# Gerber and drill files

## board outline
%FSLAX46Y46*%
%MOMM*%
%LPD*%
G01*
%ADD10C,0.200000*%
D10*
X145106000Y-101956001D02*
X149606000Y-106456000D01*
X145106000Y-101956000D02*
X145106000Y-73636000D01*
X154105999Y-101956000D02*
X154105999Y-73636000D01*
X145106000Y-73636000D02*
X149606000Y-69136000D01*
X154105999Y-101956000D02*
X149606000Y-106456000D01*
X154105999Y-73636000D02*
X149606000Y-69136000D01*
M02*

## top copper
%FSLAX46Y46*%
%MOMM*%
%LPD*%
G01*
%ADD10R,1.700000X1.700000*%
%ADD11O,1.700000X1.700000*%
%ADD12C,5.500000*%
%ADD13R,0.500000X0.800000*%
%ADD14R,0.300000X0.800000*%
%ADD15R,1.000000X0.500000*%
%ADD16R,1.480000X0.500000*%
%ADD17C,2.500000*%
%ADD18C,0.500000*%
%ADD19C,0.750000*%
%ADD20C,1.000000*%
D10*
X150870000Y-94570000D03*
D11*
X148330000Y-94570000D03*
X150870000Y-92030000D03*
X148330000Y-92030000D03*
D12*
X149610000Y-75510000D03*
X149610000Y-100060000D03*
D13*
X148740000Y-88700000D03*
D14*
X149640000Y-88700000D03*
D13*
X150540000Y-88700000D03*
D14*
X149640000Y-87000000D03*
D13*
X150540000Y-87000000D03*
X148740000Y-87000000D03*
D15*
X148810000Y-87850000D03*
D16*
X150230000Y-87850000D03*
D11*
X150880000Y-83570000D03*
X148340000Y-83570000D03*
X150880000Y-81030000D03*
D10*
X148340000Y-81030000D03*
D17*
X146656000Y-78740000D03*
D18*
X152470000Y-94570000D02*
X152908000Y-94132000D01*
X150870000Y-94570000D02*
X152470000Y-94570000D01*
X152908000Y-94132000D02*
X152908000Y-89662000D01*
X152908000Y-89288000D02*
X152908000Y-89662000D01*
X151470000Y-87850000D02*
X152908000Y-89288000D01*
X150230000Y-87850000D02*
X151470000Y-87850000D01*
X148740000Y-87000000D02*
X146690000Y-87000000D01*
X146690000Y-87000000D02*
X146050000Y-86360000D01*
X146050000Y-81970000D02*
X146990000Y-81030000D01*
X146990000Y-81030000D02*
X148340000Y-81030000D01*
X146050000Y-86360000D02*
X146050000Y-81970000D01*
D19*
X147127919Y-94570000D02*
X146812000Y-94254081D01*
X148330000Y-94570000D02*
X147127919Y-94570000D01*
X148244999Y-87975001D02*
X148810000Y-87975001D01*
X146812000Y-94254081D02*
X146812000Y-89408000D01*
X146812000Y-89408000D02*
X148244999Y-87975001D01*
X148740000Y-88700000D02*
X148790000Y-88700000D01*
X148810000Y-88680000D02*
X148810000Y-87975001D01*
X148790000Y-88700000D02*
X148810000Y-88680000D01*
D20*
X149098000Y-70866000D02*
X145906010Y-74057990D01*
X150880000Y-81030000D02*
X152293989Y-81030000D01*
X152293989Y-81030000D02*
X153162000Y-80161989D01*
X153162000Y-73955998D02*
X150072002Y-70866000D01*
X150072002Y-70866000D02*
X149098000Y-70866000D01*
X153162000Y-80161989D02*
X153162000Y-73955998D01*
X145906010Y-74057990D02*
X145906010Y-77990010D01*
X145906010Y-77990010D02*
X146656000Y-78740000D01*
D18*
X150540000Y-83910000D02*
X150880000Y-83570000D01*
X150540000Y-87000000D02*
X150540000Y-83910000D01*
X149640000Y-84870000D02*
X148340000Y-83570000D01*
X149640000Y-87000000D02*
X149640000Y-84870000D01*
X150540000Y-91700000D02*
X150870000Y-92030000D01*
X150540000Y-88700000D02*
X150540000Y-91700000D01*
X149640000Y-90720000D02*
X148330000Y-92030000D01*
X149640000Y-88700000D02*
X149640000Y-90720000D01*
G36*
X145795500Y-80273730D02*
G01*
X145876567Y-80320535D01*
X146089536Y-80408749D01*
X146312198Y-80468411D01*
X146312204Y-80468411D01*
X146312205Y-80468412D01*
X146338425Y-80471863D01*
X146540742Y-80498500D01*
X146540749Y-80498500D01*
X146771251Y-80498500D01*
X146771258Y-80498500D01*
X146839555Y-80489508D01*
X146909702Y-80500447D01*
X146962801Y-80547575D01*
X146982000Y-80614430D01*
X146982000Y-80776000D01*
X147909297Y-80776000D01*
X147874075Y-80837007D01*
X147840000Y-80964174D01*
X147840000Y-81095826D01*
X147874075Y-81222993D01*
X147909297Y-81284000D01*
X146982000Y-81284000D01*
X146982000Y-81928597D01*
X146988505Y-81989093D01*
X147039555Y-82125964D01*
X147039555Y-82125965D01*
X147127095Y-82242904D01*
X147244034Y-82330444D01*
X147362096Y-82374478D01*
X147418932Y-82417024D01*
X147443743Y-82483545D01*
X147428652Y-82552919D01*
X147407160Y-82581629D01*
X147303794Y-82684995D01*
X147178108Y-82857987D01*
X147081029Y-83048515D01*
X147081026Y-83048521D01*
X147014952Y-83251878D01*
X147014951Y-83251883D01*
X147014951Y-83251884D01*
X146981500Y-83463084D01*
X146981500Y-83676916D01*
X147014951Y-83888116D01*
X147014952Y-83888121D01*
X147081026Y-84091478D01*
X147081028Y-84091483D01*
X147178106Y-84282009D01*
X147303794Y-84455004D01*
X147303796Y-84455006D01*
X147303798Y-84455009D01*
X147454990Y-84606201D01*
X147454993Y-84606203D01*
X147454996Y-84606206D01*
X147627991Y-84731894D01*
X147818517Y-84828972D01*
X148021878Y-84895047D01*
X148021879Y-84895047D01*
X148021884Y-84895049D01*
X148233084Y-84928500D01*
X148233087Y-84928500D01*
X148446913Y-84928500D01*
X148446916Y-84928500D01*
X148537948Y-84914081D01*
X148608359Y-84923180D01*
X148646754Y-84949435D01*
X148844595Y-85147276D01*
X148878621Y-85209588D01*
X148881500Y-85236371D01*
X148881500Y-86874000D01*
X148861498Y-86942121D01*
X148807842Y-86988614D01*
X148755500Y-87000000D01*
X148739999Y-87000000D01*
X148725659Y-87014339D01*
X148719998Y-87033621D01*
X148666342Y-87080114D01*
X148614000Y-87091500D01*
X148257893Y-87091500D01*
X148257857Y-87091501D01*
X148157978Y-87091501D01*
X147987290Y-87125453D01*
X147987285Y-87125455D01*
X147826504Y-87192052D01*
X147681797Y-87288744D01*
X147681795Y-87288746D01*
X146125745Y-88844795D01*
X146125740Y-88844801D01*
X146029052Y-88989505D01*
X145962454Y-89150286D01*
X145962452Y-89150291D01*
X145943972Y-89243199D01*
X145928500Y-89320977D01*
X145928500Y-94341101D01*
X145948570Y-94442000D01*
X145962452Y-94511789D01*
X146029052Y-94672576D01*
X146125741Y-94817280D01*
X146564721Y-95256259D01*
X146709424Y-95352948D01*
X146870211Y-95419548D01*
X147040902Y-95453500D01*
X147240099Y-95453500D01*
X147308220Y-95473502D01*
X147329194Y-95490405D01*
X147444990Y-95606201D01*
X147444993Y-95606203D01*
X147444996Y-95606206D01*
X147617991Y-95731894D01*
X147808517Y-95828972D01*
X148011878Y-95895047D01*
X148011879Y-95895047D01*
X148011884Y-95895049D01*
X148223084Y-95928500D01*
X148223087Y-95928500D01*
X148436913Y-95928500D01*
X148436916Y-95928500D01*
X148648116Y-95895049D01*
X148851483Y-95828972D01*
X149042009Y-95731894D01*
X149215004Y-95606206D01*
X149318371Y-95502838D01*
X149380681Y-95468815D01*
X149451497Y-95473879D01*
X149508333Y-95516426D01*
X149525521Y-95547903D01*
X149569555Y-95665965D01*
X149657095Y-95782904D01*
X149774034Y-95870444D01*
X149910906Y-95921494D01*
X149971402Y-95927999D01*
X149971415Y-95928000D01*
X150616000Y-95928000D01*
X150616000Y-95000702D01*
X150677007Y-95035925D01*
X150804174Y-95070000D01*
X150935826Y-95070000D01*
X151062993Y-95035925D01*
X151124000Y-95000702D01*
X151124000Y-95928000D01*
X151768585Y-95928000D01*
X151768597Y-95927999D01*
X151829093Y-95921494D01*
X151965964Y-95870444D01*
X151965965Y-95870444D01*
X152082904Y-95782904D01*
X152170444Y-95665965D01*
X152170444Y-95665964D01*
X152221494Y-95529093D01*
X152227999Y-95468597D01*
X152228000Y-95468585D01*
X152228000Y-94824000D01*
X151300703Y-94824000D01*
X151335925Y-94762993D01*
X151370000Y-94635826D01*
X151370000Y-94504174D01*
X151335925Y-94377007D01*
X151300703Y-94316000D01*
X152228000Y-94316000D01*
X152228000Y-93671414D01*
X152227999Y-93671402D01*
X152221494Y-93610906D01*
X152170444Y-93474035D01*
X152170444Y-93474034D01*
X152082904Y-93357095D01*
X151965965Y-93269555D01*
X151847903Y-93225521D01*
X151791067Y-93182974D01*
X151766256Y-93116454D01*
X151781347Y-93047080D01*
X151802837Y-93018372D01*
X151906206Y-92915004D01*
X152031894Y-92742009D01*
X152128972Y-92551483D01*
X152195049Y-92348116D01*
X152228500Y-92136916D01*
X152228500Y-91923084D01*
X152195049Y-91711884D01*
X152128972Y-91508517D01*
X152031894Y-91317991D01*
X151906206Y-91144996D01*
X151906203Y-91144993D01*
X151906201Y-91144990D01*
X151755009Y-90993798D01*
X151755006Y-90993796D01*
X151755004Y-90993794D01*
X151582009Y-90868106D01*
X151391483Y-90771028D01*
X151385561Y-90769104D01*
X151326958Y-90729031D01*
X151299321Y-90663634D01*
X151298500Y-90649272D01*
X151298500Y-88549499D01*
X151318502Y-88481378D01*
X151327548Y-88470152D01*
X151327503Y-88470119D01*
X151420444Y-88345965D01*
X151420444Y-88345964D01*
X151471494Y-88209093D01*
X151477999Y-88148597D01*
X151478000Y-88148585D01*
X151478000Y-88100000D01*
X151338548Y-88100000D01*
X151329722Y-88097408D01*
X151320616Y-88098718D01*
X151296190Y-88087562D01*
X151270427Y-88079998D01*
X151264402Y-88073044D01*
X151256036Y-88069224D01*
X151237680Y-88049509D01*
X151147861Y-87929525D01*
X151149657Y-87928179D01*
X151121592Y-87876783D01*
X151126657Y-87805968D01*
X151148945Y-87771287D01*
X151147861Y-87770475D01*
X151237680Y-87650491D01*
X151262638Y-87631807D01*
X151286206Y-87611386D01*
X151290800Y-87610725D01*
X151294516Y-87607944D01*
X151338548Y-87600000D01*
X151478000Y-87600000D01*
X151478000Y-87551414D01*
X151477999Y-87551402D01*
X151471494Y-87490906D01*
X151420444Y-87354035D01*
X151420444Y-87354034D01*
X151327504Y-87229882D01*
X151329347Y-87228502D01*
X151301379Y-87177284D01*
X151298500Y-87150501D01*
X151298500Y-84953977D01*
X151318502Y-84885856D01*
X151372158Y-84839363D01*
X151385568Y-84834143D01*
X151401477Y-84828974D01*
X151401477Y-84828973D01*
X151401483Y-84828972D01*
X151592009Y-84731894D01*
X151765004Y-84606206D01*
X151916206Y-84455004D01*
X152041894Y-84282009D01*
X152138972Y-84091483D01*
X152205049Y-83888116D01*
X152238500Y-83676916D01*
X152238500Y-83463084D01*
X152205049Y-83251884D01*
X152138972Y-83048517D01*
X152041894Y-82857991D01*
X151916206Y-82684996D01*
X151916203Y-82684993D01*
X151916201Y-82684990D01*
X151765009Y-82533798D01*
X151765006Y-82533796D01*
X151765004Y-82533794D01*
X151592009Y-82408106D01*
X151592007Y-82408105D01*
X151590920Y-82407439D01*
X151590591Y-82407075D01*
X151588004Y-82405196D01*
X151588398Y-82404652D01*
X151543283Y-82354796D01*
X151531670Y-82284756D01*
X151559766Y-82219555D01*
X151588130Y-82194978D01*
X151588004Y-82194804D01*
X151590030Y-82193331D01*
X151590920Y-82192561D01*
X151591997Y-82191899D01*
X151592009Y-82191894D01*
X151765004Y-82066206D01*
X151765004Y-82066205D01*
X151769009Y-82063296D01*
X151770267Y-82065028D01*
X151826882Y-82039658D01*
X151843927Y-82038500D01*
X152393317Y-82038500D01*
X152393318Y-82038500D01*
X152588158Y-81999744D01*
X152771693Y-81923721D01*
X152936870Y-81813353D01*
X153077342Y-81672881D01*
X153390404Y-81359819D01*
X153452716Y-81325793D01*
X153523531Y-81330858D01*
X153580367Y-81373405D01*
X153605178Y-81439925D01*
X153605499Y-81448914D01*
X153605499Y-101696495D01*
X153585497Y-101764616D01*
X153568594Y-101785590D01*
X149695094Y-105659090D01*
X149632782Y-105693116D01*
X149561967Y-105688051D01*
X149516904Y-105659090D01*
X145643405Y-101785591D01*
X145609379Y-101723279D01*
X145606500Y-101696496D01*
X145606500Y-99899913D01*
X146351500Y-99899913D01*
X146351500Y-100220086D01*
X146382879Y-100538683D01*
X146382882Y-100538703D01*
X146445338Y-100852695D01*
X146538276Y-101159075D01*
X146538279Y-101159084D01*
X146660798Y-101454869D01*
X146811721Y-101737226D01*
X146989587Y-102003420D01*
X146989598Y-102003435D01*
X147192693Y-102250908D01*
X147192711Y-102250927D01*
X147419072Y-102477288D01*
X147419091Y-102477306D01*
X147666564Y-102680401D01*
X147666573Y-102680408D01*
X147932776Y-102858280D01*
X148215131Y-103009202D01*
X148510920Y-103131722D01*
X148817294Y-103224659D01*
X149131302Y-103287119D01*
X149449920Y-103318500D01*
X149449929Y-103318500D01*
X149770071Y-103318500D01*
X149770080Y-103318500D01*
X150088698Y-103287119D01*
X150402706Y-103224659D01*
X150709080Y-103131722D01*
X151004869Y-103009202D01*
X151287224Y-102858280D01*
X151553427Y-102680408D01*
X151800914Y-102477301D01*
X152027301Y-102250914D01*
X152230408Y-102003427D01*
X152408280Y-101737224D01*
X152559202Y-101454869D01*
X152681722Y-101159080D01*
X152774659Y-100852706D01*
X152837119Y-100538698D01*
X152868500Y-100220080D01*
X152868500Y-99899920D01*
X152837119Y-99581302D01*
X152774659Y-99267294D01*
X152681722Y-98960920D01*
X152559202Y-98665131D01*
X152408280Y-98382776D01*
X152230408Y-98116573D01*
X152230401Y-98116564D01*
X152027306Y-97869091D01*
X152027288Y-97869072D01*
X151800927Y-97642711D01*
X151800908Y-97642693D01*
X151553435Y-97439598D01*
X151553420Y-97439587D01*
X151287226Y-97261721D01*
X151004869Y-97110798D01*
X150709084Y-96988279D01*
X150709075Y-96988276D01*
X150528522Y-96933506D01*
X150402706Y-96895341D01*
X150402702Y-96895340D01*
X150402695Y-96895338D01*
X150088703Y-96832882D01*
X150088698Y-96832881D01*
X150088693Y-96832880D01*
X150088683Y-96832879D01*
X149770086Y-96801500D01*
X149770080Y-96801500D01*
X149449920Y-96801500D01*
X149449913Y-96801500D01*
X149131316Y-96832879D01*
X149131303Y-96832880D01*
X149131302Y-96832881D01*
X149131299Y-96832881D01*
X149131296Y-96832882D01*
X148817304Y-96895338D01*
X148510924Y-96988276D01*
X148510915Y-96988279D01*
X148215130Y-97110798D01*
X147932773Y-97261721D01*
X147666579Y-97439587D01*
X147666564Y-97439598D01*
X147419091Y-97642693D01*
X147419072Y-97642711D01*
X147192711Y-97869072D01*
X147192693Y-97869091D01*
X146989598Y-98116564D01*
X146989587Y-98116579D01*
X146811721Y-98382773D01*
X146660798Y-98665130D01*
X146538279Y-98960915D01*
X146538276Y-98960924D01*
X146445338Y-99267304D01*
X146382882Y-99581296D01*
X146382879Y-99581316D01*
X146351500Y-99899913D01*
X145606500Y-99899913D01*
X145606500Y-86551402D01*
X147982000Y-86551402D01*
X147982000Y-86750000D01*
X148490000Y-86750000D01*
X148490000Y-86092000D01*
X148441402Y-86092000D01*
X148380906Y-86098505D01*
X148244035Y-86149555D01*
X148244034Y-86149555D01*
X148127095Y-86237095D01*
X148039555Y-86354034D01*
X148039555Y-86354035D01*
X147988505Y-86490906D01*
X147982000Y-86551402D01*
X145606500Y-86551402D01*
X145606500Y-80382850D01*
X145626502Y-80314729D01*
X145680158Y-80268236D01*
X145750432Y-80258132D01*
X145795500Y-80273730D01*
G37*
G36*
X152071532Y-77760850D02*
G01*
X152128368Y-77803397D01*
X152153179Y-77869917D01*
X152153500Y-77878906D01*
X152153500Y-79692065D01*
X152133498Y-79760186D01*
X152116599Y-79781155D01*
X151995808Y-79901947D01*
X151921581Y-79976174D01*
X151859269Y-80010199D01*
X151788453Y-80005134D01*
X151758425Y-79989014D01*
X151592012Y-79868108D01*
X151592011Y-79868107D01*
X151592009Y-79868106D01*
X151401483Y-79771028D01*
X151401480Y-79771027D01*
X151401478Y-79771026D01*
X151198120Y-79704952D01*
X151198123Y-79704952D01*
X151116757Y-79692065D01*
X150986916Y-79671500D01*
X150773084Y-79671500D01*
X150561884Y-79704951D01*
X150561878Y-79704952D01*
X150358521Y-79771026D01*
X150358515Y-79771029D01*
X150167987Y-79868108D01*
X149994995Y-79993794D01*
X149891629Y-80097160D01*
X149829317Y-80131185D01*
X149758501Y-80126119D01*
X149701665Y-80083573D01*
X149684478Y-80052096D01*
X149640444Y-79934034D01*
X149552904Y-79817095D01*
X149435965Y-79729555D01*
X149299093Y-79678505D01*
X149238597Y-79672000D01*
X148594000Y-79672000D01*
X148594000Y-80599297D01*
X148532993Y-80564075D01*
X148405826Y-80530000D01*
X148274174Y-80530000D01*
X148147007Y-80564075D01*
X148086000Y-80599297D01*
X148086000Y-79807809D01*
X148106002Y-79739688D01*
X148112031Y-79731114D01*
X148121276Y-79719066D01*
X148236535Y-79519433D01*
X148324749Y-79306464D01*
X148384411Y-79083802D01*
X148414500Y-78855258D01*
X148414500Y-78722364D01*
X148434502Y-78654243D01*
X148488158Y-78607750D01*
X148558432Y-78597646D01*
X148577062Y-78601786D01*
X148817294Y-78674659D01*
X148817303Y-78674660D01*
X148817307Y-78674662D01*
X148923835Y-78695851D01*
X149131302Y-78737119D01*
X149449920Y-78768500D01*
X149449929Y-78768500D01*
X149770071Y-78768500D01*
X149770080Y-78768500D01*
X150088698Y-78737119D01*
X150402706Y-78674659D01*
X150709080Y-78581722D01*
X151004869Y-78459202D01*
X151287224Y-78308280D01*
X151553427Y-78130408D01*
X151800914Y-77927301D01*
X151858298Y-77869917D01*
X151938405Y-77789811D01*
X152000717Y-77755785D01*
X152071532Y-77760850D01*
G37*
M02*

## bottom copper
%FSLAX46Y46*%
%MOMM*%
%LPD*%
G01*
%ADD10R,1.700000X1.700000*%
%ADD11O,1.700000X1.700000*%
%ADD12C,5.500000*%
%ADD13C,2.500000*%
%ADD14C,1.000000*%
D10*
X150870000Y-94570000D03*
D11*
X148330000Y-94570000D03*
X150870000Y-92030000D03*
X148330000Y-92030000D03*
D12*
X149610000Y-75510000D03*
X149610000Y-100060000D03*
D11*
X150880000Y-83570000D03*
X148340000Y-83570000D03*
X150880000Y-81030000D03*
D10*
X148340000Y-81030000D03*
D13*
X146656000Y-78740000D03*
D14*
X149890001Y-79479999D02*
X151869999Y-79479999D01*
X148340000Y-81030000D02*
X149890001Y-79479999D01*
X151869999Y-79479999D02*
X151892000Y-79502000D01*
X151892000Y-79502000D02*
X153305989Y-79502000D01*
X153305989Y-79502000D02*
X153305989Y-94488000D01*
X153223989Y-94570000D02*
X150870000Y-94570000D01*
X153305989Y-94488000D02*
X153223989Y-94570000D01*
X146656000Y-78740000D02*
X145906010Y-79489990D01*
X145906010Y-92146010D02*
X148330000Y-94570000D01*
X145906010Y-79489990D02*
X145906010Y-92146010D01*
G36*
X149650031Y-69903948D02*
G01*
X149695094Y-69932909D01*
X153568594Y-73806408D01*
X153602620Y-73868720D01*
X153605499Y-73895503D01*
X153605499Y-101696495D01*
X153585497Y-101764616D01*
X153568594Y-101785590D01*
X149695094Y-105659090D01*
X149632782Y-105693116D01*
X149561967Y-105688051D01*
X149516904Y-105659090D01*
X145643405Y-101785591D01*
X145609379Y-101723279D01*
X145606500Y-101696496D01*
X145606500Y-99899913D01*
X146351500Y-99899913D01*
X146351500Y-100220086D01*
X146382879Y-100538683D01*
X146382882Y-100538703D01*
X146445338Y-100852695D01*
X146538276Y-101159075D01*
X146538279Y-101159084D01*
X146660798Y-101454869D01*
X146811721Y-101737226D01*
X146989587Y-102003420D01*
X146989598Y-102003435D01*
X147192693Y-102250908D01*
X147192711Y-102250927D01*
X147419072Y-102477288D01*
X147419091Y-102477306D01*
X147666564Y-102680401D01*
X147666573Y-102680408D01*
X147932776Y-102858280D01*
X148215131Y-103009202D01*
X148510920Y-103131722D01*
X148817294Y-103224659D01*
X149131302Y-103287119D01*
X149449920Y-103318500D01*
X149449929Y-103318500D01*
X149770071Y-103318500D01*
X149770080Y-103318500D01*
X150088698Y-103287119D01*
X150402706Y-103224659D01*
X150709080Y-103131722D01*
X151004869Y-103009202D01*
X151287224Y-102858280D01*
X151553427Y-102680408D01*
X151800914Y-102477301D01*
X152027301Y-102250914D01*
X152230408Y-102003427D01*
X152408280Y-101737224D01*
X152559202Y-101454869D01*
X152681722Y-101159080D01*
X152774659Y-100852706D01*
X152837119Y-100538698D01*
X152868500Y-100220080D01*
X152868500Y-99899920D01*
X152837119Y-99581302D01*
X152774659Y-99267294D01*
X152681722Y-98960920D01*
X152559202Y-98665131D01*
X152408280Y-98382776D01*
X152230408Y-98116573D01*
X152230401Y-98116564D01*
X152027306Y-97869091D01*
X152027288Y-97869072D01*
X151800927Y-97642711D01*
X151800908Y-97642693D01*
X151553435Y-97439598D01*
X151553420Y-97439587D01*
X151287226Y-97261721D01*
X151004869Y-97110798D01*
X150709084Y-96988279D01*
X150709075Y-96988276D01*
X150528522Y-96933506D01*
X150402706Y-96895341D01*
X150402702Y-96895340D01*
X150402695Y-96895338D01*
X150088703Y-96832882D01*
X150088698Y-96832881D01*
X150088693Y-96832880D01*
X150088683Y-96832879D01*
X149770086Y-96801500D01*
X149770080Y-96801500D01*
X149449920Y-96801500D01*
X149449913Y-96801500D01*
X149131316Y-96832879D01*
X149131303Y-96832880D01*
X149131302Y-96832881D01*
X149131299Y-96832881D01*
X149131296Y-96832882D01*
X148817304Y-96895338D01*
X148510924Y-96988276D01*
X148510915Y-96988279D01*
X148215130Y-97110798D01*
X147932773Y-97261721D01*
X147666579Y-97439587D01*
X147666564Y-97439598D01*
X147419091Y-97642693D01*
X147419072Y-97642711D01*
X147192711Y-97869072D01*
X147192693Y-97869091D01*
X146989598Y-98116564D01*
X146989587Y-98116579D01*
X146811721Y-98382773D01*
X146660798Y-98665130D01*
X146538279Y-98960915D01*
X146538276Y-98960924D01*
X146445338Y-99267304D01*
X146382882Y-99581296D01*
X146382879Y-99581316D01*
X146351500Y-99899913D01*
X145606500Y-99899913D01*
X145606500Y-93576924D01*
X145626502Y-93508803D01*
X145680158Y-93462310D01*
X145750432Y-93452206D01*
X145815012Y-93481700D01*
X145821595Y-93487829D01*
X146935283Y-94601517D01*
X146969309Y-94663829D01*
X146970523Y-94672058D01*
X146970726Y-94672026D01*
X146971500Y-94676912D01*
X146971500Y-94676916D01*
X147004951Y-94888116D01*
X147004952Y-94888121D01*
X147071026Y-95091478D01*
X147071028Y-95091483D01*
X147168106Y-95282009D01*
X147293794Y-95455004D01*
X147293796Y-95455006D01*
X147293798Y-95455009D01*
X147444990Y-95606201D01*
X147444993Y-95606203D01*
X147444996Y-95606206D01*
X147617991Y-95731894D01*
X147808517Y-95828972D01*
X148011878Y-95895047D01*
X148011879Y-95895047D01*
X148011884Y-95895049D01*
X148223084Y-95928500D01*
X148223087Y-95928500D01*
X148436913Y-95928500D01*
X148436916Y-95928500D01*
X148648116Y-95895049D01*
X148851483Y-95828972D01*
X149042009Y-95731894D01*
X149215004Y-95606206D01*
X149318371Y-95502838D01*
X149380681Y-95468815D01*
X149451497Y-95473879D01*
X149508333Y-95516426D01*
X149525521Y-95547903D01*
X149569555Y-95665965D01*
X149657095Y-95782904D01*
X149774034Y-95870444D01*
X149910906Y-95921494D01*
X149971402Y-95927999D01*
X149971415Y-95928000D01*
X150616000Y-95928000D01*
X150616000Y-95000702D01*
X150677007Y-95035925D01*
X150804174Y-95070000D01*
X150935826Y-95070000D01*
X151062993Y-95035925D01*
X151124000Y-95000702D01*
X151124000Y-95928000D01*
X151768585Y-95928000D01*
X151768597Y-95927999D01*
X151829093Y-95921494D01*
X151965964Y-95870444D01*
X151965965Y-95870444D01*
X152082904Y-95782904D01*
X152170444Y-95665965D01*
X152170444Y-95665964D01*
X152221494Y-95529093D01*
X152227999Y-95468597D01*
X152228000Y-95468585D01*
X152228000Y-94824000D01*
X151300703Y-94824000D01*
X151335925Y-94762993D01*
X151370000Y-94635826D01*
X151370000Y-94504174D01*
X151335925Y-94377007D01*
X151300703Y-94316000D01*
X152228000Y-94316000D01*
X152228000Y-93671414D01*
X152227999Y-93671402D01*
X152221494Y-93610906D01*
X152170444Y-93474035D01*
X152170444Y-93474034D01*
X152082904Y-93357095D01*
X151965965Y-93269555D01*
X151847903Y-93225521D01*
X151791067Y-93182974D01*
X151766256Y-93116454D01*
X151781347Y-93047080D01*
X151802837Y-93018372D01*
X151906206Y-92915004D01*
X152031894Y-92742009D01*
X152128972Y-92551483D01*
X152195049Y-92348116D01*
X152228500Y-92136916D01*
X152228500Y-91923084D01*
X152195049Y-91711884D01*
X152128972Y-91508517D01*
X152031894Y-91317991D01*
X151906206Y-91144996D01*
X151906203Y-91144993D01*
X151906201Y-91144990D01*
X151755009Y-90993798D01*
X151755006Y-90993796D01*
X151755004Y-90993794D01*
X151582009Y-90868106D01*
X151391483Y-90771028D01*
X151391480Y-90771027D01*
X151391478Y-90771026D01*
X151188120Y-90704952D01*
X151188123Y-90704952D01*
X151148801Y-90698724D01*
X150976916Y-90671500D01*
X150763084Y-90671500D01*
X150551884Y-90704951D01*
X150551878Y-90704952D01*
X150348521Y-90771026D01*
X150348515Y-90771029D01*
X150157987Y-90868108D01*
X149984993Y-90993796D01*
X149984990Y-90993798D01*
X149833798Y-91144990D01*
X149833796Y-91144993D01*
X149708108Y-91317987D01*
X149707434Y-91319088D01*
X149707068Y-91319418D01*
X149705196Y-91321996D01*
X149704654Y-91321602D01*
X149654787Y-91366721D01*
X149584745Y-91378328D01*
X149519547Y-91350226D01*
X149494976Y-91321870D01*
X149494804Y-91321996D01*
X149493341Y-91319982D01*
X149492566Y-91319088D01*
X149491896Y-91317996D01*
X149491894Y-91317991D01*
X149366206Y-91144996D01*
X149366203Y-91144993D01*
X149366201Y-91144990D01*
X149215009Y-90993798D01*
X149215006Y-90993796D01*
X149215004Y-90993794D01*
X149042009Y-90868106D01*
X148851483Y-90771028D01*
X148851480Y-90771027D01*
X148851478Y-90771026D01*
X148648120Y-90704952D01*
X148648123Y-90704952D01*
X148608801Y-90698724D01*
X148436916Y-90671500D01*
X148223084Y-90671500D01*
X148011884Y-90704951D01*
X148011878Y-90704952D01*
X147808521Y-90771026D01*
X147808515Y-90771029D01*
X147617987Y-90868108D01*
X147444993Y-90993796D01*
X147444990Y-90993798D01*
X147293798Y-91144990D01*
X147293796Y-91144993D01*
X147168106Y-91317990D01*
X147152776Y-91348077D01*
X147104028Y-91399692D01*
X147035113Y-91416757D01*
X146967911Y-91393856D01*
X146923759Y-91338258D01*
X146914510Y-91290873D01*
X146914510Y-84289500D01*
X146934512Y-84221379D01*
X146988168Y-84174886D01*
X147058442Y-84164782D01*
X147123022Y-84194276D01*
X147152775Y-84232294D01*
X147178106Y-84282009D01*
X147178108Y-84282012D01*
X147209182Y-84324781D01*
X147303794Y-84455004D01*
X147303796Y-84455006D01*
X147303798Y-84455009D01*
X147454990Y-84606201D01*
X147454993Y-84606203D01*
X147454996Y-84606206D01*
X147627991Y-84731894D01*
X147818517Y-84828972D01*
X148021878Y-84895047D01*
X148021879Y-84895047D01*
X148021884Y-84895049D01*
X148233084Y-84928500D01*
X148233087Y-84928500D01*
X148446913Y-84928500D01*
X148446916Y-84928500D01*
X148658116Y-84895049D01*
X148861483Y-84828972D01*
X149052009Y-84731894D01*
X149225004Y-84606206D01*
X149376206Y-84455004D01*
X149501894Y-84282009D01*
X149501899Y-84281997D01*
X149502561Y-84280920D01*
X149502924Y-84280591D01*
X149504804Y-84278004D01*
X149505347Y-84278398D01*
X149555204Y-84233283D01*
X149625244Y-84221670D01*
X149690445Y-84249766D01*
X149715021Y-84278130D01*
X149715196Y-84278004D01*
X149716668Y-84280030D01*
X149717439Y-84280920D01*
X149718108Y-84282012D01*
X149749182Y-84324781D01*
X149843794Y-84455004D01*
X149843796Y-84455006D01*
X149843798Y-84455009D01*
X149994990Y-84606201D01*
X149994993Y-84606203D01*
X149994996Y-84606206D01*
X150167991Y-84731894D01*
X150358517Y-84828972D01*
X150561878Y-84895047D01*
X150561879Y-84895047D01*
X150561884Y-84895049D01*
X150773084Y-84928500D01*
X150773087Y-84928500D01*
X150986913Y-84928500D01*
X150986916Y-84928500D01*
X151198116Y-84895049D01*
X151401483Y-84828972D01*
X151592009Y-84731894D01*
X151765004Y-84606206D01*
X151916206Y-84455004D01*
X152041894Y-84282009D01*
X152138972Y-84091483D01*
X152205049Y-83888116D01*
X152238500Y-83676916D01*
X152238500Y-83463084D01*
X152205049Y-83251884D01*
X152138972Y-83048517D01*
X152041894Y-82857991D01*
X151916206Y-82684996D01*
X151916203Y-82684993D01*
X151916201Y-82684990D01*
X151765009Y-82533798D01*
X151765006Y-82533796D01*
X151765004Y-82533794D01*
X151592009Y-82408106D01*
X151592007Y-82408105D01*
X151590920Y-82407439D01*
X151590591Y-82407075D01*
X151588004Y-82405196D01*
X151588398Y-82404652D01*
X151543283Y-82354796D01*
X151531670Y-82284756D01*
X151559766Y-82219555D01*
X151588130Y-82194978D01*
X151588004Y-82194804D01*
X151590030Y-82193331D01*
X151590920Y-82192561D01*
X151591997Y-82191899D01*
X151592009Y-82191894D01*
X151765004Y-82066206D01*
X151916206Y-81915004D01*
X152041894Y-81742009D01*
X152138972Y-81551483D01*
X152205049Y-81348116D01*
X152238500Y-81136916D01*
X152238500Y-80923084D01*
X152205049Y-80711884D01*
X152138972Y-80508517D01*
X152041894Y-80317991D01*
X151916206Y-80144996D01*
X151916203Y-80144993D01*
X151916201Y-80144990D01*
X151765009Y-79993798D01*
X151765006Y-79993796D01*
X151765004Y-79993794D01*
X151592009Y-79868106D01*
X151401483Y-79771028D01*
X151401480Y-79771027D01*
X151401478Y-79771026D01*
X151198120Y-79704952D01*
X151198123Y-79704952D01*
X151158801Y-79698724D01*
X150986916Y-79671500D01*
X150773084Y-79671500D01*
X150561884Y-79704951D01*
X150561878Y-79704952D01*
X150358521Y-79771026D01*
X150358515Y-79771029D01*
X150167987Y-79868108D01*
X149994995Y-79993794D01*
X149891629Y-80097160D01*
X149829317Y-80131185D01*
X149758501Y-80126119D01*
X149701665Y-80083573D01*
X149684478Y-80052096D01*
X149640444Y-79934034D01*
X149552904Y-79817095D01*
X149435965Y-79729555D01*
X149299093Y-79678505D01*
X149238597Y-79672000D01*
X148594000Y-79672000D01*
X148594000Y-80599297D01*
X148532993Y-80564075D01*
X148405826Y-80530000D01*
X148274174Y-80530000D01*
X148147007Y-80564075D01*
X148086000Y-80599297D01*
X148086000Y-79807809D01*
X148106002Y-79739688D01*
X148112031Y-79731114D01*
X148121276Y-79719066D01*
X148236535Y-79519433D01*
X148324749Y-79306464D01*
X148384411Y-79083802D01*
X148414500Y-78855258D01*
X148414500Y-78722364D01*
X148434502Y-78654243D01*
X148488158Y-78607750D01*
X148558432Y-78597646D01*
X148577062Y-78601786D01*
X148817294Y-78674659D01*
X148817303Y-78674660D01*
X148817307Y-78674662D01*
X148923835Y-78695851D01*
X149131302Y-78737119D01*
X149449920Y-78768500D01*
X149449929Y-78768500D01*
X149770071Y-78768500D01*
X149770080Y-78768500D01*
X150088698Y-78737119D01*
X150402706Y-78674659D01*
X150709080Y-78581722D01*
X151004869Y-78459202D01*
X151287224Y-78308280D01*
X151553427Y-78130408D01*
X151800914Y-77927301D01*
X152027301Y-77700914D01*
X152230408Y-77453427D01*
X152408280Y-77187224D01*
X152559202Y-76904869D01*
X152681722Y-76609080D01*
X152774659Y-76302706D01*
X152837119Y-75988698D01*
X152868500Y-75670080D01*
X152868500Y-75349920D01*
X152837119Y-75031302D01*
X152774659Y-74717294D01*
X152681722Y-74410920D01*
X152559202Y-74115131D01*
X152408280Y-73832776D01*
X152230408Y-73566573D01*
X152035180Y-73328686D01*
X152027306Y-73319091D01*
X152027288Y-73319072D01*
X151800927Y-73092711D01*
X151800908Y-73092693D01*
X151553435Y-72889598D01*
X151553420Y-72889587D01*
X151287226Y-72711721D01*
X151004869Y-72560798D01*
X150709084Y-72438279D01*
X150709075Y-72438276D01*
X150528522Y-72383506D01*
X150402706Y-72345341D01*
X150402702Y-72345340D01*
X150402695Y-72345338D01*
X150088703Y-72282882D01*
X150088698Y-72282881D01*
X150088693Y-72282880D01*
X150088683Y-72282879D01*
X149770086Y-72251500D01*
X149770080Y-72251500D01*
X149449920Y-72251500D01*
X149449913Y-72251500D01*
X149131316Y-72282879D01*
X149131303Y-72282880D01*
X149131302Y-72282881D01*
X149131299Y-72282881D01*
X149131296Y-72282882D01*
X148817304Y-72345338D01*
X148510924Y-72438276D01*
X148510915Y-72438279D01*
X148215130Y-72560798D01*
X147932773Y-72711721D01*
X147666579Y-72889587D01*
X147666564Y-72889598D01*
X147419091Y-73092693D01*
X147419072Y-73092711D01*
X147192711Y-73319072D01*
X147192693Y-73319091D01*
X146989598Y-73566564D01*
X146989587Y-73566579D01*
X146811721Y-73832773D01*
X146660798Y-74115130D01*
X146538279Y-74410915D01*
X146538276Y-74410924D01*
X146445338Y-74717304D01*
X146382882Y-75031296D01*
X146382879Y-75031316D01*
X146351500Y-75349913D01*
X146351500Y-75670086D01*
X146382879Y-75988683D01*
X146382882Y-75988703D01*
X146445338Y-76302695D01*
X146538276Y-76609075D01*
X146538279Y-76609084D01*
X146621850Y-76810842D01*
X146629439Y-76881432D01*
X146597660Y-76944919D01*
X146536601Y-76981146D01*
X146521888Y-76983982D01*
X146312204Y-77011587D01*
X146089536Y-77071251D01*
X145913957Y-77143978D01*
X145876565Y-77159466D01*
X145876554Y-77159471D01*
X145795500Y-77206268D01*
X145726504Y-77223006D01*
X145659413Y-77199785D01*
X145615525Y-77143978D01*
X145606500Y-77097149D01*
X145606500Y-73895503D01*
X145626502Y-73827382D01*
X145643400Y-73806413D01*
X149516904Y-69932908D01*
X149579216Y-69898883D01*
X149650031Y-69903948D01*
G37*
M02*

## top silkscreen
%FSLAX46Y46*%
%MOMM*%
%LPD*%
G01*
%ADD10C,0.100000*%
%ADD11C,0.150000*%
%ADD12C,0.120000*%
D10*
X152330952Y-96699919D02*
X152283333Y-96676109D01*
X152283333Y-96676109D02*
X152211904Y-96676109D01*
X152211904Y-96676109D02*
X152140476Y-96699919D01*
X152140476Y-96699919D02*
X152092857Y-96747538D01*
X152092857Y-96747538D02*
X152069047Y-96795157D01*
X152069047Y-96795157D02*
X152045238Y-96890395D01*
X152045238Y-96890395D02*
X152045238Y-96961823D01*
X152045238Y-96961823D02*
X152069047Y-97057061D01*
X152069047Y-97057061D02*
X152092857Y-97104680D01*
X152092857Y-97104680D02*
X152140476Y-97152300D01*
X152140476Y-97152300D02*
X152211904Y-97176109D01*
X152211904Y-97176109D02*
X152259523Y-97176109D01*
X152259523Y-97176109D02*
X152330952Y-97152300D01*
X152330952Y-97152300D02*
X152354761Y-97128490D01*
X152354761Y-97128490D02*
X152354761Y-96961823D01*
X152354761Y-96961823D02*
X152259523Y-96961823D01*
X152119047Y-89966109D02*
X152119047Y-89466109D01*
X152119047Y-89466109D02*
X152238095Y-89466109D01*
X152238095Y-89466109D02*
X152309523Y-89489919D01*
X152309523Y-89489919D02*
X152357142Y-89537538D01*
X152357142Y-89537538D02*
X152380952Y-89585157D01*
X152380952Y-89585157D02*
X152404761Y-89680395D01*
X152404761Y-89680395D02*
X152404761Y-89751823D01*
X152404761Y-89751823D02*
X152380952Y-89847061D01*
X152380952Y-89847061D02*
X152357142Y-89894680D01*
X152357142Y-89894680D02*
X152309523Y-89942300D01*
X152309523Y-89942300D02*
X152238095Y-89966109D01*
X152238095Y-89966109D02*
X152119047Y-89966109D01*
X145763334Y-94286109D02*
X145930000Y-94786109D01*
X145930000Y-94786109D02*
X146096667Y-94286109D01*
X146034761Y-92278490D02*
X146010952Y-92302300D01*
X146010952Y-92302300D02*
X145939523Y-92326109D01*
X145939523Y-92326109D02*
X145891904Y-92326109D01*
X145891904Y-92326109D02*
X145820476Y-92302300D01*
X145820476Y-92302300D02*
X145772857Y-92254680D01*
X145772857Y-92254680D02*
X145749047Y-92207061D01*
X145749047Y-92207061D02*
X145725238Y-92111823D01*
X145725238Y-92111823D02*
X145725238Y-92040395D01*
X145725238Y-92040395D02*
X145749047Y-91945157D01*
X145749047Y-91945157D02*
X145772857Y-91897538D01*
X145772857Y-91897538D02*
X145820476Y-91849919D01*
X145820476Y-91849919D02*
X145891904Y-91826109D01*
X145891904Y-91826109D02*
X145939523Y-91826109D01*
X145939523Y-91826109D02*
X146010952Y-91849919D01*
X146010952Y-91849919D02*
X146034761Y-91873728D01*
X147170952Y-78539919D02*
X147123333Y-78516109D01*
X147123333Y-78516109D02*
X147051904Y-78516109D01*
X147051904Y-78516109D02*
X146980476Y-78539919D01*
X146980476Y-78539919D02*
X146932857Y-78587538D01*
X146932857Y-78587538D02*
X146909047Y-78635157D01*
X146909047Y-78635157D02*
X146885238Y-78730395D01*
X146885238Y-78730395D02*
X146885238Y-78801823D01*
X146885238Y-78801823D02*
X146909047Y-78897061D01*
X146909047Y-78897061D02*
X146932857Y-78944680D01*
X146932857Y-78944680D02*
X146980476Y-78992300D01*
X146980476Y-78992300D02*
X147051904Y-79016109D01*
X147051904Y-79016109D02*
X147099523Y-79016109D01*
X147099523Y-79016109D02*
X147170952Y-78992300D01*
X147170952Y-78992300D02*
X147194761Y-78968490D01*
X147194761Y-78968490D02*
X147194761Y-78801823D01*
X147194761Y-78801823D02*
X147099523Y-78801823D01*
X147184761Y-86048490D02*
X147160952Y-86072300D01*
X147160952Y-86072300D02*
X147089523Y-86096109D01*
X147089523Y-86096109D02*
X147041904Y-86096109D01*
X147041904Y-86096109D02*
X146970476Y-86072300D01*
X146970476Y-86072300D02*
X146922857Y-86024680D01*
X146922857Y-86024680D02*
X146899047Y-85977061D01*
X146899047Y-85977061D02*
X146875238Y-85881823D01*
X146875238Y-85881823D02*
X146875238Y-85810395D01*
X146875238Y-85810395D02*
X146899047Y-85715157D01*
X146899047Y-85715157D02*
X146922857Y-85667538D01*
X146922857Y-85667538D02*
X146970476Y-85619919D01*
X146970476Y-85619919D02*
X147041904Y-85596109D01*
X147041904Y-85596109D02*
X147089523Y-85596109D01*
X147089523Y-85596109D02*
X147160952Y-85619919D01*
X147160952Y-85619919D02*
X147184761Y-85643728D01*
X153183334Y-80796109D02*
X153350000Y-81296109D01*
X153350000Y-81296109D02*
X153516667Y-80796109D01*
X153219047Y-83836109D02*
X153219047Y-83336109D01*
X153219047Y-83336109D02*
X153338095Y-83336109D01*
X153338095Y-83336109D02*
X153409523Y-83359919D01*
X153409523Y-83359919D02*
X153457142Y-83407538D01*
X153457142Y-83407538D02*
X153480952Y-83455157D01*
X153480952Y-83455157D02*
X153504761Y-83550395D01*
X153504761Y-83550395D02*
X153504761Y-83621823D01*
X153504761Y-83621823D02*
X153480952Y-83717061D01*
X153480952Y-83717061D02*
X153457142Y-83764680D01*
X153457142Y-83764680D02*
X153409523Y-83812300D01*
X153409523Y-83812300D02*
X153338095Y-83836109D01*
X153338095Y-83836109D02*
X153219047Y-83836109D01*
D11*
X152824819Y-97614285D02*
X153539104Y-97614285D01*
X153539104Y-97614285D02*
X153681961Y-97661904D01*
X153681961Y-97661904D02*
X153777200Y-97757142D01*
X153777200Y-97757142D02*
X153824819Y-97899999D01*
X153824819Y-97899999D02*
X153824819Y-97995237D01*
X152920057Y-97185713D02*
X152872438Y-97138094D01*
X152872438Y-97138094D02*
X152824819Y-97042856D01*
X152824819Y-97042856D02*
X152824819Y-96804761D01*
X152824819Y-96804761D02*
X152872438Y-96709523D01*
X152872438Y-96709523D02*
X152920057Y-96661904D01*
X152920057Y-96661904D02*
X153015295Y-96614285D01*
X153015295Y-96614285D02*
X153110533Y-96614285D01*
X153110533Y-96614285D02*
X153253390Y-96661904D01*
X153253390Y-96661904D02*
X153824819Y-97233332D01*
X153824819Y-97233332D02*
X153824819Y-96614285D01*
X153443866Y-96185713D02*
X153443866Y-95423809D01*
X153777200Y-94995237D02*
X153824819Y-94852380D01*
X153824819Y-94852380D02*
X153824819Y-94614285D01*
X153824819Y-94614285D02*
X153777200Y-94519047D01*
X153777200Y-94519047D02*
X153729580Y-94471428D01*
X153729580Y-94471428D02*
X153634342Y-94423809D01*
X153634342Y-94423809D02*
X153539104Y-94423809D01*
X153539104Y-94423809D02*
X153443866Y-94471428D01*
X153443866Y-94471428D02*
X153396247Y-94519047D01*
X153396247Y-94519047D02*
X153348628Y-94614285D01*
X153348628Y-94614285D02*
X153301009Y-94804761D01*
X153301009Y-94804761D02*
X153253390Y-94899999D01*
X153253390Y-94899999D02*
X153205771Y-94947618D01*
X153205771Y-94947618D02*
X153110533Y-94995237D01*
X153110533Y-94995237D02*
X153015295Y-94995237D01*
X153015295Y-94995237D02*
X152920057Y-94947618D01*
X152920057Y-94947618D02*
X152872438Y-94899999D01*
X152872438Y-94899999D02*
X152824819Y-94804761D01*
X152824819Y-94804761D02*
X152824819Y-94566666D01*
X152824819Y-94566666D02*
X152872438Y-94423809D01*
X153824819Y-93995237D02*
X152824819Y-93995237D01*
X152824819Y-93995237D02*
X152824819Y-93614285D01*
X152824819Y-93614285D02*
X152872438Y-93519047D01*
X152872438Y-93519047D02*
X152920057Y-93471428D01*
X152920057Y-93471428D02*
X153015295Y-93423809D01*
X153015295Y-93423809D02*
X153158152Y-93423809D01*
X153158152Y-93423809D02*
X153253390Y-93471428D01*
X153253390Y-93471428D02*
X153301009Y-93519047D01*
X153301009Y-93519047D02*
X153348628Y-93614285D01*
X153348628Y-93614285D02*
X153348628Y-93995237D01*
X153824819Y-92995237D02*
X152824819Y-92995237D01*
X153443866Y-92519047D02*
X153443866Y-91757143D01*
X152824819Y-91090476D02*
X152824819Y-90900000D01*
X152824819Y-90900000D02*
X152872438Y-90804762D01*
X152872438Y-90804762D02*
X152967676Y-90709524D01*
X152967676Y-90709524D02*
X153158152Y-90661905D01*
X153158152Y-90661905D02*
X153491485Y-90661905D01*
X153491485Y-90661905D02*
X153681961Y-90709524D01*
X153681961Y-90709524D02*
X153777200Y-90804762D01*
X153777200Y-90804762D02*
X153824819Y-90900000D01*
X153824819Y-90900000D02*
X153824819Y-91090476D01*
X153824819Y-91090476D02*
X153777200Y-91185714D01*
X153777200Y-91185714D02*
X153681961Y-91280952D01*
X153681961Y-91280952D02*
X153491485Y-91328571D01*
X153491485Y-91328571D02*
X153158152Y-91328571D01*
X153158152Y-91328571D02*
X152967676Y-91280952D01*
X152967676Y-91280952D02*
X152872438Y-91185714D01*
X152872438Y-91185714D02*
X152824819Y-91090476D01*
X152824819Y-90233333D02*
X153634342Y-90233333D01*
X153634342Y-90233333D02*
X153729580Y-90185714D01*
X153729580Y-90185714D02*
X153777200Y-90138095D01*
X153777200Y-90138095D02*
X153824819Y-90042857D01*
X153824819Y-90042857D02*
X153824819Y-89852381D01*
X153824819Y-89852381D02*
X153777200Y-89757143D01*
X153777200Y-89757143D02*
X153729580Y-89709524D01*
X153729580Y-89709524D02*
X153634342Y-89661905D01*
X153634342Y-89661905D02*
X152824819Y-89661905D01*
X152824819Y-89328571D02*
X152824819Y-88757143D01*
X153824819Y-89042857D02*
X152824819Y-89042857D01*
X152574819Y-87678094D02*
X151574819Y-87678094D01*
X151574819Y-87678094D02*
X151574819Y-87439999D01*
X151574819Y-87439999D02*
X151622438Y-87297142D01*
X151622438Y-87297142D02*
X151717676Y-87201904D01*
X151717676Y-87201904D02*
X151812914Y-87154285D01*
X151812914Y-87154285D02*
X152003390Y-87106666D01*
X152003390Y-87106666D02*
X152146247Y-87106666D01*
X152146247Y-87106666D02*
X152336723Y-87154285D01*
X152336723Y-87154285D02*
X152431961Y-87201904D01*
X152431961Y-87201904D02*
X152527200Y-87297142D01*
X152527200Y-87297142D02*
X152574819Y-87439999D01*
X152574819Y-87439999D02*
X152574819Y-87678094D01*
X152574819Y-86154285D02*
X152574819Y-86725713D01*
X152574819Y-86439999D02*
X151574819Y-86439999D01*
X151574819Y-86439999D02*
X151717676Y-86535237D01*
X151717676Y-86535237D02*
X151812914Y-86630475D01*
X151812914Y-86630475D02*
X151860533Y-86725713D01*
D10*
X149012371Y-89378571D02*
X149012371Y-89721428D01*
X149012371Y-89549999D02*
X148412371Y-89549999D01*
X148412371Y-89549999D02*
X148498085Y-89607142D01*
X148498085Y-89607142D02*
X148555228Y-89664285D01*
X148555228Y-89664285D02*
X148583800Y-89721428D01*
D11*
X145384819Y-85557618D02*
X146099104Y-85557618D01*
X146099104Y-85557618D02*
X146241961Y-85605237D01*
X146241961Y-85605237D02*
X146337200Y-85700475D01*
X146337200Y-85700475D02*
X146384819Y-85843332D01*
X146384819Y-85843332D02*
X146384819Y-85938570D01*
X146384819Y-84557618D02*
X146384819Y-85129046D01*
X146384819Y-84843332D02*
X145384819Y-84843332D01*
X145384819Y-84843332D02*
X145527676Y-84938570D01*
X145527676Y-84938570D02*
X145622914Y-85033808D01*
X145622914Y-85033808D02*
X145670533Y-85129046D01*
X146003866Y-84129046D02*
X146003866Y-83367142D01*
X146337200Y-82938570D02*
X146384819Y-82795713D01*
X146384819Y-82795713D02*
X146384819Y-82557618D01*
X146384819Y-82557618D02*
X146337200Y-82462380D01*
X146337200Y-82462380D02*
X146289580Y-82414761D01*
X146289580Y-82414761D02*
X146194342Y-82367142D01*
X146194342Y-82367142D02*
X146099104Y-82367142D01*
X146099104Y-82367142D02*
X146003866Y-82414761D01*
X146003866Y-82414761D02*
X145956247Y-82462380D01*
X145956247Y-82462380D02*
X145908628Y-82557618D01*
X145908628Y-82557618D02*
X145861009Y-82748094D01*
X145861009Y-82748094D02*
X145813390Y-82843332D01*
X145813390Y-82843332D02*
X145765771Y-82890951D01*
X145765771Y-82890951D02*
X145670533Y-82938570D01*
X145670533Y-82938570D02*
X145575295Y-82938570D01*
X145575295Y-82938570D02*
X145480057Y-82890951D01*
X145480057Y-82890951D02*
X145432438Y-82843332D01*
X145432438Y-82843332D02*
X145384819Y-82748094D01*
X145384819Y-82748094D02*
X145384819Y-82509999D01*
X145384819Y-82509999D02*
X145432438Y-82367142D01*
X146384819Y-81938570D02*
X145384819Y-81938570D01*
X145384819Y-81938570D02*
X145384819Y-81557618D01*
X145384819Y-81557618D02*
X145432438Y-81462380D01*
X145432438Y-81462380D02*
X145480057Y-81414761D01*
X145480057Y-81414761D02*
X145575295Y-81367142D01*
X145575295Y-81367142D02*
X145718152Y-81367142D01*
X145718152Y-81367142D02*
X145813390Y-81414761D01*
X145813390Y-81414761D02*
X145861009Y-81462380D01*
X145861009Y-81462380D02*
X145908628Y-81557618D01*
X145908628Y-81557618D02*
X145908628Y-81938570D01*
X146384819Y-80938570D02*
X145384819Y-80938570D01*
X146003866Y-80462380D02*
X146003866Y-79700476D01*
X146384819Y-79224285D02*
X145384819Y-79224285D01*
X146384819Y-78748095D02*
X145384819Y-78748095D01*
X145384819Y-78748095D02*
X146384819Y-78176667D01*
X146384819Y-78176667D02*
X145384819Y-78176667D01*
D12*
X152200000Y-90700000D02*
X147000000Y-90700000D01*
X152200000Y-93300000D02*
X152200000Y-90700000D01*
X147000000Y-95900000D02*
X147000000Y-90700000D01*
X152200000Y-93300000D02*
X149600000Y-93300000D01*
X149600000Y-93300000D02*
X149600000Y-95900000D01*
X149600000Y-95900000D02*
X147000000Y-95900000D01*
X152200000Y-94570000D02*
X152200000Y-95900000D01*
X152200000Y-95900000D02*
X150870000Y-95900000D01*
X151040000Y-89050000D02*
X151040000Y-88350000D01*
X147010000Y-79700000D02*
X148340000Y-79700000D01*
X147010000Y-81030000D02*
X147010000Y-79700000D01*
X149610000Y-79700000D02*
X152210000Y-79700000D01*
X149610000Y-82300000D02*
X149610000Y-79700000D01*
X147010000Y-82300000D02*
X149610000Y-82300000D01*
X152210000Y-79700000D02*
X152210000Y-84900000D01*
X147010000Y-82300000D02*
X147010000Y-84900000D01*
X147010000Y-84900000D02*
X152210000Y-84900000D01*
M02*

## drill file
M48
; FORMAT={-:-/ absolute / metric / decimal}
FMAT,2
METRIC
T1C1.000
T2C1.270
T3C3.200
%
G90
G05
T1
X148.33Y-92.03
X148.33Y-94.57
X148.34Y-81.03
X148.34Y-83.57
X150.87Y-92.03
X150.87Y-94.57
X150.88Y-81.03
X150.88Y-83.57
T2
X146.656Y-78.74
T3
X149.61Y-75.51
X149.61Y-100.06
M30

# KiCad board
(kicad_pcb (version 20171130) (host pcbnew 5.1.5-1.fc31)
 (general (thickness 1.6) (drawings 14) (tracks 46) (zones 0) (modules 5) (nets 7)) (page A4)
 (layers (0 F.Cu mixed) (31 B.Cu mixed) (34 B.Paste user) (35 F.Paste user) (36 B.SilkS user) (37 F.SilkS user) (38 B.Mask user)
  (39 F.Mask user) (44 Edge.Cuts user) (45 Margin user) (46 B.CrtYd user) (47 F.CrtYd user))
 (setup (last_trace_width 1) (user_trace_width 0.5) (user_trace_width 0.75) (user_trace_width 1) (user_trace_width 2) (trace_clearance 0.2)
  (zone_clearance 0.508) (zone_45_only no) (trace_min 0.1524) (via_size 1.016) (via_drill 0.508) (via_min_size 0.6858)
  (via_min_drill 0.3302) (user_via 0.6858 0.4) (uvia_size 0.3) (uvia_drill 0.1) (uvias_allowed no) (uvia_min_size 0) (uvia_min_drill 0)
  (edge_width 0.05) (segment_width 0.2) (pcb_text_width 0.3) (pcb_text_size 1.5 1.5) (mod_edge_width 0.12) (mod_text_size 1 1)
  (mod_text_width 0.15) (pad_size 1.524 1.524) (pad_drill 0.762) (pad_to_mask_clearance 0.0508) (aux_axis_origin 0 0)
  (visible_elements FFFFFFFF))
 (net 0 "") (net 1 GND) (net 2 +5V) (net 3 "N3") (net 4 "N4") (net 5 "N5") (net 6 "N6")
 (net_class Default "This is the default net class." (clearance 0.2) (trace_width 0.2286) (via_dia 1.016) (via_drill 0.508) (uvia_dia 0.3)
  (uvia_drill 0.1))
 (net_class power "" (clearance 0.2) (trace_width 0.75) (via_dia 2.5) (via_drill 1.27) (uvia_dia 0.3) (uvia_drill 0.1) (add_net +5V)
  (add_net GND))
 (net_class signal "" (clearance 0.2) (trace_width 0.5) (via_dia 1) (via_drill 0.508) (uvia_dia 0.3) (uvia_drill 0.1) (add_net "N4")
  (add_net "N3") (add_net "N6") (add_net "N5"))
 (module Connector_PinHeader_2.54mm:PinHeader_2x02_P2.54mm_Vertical (layer F.Cu) (at 150.87 94.57 180)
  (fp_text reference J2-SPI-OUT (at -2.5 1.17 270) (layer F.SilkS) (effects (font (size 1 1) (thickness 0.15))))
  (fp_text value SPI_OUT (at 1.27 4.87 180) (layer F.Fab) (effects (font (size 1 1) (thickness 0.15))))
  (fp_line (start -1.33 3.87) (end 3.87 3.87) (layer F.SilkS) (width 0.12))
  (fp_line (start -1.33 1.27) (end -1.33 3.87) (layer F.SilkS) (width 0.12))
  (fp_line (start 3.87 -1.33) (end 3.87 3.87) (layer F.SilkS) (width 0.12))
  (fp_line (start -1.33 1.27) (end 1.27 1.27) (layer F.SilkS) (width 0.12))
  (fp_line (start 1.27 1.27) (end 1.27 -1.33) (layer F.SilkS) (width 0.12))
  (fp_line (start 1.27 -1.33) (end 3.87 -1.33) (layer F.SilkS) (width 0.12))
  (fp_line (start -1.33 0) (end -1.33 -1.33) (layer F.SilkS) (width 0.12))
  (fp_line (start -1.33 -1.33) (end 0 -1.33) (layer F.SilkS) (width 0.12))
  (pad 1 thru_hole rect (at 0 0 180) (size 1.7 1.7) (drill 1) (layers *.Cu *.Mask) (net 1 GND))
  (pad 2 thru_hole oval (at 2.54 0 180) (size 1.7 1.7) (drill 1) (layers *.Cu *.Mask) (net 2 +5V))
  (pad 3 thru_hole oval (at 0 2.54 180) (size 1.7 1.7) (drill 1) (layers *.Cu *.Mask) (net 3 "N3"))
  (pad 4 thru_hole oval (at 2.54 2.54 180) (size 1.7 1.7) (drill 1) (layers *.Cu *.Mask) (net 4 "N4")))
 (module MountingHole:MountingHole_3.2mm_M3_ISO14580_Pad (layer F.Cu) (at 149.61 75.51)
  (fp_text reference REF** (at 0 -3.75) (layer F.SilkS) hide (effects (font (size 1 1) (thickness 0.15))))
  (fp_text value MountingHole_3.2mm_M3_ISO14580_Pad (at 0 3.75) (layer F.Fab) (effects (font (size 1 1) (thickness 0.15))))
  (pad 1 thru_hole circle (at 0 0) (size 5.5 5.5) (drill 3.2) (layers *.Cu *.Mask)))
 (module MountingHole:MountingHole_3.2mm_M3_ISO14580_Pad (layer F.Cu) (at 149.61 100.06)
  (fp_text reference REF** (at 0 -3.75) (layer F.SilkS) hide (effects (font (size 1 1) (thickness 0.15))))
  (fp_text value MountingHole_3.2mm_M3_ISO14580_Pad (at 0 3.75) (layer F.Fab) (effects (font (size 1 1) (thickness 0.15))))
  (pad 1 thru_hole circle (at 0 0) (size 5.5 5.5) (drill 3.2) (layers *.Cu *.Mask)))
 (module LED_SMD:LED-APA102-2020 (layer F.Cu) (at 149.64 87.85 90)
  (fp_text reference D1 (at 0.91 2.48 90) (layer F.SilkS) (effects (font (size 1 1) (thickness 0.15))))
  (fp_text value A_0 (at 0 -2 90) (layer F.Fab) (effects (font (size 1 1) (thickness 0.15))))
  (fp_line (start -1.2 1.4) (end -0.5 1.4) (layer F.SilkS) (width 0.12))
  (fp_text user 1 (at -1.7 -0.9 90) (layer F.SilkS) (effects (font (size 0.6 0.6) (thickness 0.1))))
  (pad 1 smd rect (at -0.85 -0.9 90) (size 0.8 0.5) (layers F.Cu F.Paste F.Mask) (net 2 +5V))
  (pad 2 smd rect (at -0.85 0 90) (size 0.8 0.3) (layers F.Cu F.Paste F.Mask) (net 4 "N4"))
  (pad 3 smd rect (at -0.85 0.9 90) (size 0.8 0.5) (layers F.Cu F.Paste F.Mask) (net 3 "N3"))
  (pad 5 smd rect (at 0.85 0 90) (size 0.8 0.3) (layers F.Cu F.Paste F.Mask) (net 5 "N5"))
  (pad 4 smd rect (at 0.85 0.9 90) (size 0.8 0.5) (layers F.Cu F.Paste F.Mask) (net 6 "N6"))
  (pad 6 smd rect (at 0.85 -0.9 90) (size 0.8 0.5) (layers F.Cu F.Paste F.Mask) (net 1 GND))
  (pad 1 smd rect (at 0 -0.83 180) (size 1 0.5) (layers F.Cu F.Paste F.Mask) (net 2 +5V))
  (pad 6 smd rect (at 0 0.59 180) (size 1.48 0.5) (layers F.Cu F.Paste F.Mask) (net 1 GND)))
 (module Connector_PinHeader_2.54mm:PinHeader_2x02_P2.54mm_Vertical (layer F.Cu) (at 148.34 81.03)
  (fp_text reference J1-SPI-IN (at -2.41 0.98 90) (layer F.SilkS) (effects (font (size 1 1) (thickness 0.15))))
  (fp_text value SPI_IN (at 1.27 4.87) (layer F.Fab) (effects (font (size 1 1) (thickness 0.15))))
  (fp_line (start -1.33 -1.33) (end 0 -1.33) (layer F.SilkS) (width 0.12))
  (fp_line (start -1.33 0) (end -1.33 -1.33) (layer F.SilkS) (width 0.12))
  (fp_line (start 1.27 -1.33) (end 3.87 -1.33) (layer F.SilkS) (width 0.12))
  (fp_line (start 1.27 1.27) (end 1.27 -1.33) (layer F.SilkS) (width 0.12))
  (fp_line (start -1.33 1.27) (end 1.27 1.27) (layer F.SilkS) (width 0.12))
  (fp_line (start 3.87 -1.33) (end 3.87 3.87) (layer F.SilkS) (width 0.12))
  (fp_line (start -1.33 1.27) (end -1.33 3.87) (layer F.SilkS) (width 0.12))
  (fp_line (start -1.33 3.87) (end 3.87 3.87) (layer F.SilkS) (width 0.12))
  (pad 4 thru_hole oval (at 2.54 2.54) (size 1.7 1.7) (drill 1) (layers *.Cu *.Mask) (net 6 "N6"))
  (pad 3 thru_hole oval (at 0 2.54) (size 1.7 1.7) (drill 1) (layers *.Cu *.Mask) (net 5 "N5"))
  (pad 2 thru_hole oval (at 2.54 0) (size 1.7 1.7) (drill 1) (layers *.Cu *.Mask) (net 2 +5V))
  (pad 1 thru_hole rect (at 0 0) (size 1.7 1.7) (drill 1) (layers *.Cu *.Mask) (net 1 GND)))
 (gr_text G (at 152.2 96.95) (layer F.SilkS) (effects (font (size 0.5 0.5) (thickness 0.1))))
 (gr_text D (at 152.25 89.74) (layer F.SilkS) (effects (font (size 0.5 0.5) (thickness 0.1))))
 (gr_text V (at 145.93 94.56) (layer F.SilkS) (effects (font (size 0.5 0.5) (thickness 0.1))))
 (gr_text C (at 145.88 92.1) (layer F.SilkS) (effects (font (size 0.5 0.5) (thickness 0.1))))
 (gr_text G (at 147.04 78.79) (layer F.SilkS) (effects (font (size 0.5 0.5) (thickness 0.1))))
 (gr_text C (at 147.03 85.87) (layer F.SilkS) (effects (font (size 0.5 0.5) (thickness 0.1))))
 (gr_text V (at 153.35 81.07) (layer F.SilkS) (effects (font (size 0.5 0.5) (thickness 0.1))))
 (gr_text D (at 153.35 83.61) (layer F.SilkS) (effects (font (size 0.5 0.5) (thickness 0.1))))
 (gr_line (start 145.106 101.956001) (end 149.606 106.456) (layer Edge.Cuts) (width 0.2))
 (gr_line (start 145.106 101.956) (end 145.106 73.636) (layer Edge.Cuts) (width 0.2))
 (gr_line (start 154.105999 101.956) (end 154.105999 73.636) (layer Edge.Cuts) (width 0.2))
 (gr_line (start 145.106 73.636) (end 149.606 69.136) (layer Edge.Cuts) (width 0.2))
 (gr_line (start 154.105999 101.956) (end 149.606 106.456) (layer Edge.Cuts) (width 0.2))
 (gr_line (start 154.105999 73.636) (end 149.606 69.136) (layer Edge.Cuts) (width 0.2))
 (segment (start 152.47 94.57) (end 152.908 94.132) (width 0.5) (layer F.Cu) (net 1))
 (segment (start 150.87 94.57) (end 152.47 94.57) (width 0.5) (layer F.Cu) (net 1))
 (segment (start 152.908 94.132) (end 152.908 89.662) (width 0.5) (layer F.Cu) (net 1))
 (segment (start 152.908 89.288) (end 152.908 89.662) (width 0.5) (layer F.Cu) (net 1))
 (segment (start 151.47 87.85) (end 152.908 89.288) (width 0.5) (layer F.Cu) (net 1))
 (segment (start 150.23 87.85) (end 151.47 87.85) (width 0.5) (layer F.Cu) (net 1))
 (segment (start 148.74 87) (end 146.69 87) (width 0.5) (layer F.Cu) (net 1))
 (segment (start 146.69 87) (end 146.05 86.36) (width 0.5) (layer F.Cu) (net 1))
 (segment (start 146.05 81.97) (end 146.99 81.03) (width 0.5) (layer F.Cu) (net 1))
 (segment (start 146.99 81.03) (end 148.34 81.03) (width 0.5) (layer F.Cu) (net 1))
 (segment (start 146.05 86.36) (end 146.05 81.97) (width 0.5) (layer F.Cu) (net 1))
 (segment (start 149.890001 79.479999) (end 151.869999 79.479999) (width 1) (layer B.Cu) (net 1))
 (segment (start 148.34 81.03) (end 149.890001 79.479999) (width 1) (layer B.Cu) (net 1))
 (segment (start 151.869999 79.479999) (end 151.892 79.502) (width 1) (layer B.Cu) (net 1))
 (segment (start 151.892 79.502) (end 153.305989 79.502) (width 1) (layer B.Cu) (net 1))
 (segment (start 153.305989 79.502) (end 153.305989 94.488) (width 1) (layer B.Cu) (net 1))
 (segment (start 153.223989 94.57) (end 150.87 94.57) (width 1) (layer B.Cu) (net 1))
 (segment (start 153.305989 94.488) (end 153.223989 94.57) (width 1) (layer B.Cu) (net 1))
 (segment (start 147.127919 94.57) (end 146.812 94.254081) (width 0.75) (layer F.Cu) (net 2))
 (segment (start 148.33 94.57) (end 147.127919 94.57) (width 0.75) (layer F.Cu) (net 2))
 (segment (start 148.244999 87.975001) (end 148.81 87.975001) (width 0.75) (layer F.Cu) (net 2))
 (segment (start 146.812 94.254081) (end 146.812 89.408) (width 0.75) (layer F.Cu) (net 2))
 (segment (start 146.812 89.408) (end 148.244999 87.975001) (width 0.75) (layer F.Cu) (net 2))
 (segment (start 148.74 88.7) (end 148.79 88.7) (width 0.75) (layer F.Cu) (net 2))
 (segment (start 148.81 88.68) (end 148.81 87.975001) (width 0.75) (layer F.Cu) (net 2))
 (segment (start 148.79 88.7) (end 148.81 88.68) (width 0.75) (layer F.Cu) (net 2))
 (segment (start 149.098 70.866) (end 145.90601 74.05799) (width 1) (layer F.Cu) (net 2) (status 1000000))
 (segment (start 150.88 81.03) (end 152.293989 81.03) (width 1) (layer F.Cu) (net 2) (status 1000000))
 (segment (start 152.293989 81.03) (end 153.162 80.161989) (width 1) (layer F.Cu) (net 2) (status 1000000))
 (segment (start 153.162 73.955998) (end 150.072002 70.866) (width 1) (layer F.Cu) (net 2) (status 1000000))
 (segment (start 150.072002 70.866) (end 149.098 70.866) (width 1) (layer F.Cu) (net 2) (status 1000000))
 (segment (start 153.162 80.161989) (end 153.162 73.955998) (width 1) (layer F.Cu) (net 2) (status 1000000))
 (via (at 146.656 78.74) (size 2.5) (drill 1.27) (layers F.Cu B.Cu) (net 2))
 (segment (start 145.90601 74.05799) (end 145.90601 77.99001) (width 1) (layer F.Cu) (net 2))
 (segment (start 145.90601 77.99001) (end 146.656 78.74) (width 1) (layer F.Cu) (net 2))
 (segment (start 146.656 78.74) (end 145.90601 79.48999) (width 1) (layer B.Cu) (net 2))
 (segment (start 145.90601 92.14601) (end 148.33 94.57) (width 1) (layer B.Cu) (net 2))
 (segment (start 145.90601 79.48999) (end 145.90601 92.14601) (width 1) (layer B.Cu) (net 2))
 (segment (start 150.54 83.91) (end 150.88 83.57) (width 0.5) (layer F.Cu) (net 6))
 (segment (start 150.54 87) (end 150.54 83.91) (width 0.5) (layer F.Cu) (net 6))
 (segment (start 149.64 84.87) (end 148.34 83.57) (width 0.5) (layer F.Cu) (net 5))
 (segment (start 149.64 87) (end 149.64 84.87) (width 0.5) (layer F.Cu) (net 5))
 (segment (start 150.54 91.7) (end 150.87 92.03) (width 0.5) (layer F.Cu) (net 3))
 (segment (start 150.54 88.7) (end 150.54 91.7) (width 0.5) (layer F.Cu) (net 3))
 (segment (start 149.64 90.72) (end 148.33 92.03) (width 0.5) (layer F.Cu) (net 4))
 (segment (start 149.64 88.7) (end 149.64 90.72) (width 0.5) (layer F.Cu) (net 4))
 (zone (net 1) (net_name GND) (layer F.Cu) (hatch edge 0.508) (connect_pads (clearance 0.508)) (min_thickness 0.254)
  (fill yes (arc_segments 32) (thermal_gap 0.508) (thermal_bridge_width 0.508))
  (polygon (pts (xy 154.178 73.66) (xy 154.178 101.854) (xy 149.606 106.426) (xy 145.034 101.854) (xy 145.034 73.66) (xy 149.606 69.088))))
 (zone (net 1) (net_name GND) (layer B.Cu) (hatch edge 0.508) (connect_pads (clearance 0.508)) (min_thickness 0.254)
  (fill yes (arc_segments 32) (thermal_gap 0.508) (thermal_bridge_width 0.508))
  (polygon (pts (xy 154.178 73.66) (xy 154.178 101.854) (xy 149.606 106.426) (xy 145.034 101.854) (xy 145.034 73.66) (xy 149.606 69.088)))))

